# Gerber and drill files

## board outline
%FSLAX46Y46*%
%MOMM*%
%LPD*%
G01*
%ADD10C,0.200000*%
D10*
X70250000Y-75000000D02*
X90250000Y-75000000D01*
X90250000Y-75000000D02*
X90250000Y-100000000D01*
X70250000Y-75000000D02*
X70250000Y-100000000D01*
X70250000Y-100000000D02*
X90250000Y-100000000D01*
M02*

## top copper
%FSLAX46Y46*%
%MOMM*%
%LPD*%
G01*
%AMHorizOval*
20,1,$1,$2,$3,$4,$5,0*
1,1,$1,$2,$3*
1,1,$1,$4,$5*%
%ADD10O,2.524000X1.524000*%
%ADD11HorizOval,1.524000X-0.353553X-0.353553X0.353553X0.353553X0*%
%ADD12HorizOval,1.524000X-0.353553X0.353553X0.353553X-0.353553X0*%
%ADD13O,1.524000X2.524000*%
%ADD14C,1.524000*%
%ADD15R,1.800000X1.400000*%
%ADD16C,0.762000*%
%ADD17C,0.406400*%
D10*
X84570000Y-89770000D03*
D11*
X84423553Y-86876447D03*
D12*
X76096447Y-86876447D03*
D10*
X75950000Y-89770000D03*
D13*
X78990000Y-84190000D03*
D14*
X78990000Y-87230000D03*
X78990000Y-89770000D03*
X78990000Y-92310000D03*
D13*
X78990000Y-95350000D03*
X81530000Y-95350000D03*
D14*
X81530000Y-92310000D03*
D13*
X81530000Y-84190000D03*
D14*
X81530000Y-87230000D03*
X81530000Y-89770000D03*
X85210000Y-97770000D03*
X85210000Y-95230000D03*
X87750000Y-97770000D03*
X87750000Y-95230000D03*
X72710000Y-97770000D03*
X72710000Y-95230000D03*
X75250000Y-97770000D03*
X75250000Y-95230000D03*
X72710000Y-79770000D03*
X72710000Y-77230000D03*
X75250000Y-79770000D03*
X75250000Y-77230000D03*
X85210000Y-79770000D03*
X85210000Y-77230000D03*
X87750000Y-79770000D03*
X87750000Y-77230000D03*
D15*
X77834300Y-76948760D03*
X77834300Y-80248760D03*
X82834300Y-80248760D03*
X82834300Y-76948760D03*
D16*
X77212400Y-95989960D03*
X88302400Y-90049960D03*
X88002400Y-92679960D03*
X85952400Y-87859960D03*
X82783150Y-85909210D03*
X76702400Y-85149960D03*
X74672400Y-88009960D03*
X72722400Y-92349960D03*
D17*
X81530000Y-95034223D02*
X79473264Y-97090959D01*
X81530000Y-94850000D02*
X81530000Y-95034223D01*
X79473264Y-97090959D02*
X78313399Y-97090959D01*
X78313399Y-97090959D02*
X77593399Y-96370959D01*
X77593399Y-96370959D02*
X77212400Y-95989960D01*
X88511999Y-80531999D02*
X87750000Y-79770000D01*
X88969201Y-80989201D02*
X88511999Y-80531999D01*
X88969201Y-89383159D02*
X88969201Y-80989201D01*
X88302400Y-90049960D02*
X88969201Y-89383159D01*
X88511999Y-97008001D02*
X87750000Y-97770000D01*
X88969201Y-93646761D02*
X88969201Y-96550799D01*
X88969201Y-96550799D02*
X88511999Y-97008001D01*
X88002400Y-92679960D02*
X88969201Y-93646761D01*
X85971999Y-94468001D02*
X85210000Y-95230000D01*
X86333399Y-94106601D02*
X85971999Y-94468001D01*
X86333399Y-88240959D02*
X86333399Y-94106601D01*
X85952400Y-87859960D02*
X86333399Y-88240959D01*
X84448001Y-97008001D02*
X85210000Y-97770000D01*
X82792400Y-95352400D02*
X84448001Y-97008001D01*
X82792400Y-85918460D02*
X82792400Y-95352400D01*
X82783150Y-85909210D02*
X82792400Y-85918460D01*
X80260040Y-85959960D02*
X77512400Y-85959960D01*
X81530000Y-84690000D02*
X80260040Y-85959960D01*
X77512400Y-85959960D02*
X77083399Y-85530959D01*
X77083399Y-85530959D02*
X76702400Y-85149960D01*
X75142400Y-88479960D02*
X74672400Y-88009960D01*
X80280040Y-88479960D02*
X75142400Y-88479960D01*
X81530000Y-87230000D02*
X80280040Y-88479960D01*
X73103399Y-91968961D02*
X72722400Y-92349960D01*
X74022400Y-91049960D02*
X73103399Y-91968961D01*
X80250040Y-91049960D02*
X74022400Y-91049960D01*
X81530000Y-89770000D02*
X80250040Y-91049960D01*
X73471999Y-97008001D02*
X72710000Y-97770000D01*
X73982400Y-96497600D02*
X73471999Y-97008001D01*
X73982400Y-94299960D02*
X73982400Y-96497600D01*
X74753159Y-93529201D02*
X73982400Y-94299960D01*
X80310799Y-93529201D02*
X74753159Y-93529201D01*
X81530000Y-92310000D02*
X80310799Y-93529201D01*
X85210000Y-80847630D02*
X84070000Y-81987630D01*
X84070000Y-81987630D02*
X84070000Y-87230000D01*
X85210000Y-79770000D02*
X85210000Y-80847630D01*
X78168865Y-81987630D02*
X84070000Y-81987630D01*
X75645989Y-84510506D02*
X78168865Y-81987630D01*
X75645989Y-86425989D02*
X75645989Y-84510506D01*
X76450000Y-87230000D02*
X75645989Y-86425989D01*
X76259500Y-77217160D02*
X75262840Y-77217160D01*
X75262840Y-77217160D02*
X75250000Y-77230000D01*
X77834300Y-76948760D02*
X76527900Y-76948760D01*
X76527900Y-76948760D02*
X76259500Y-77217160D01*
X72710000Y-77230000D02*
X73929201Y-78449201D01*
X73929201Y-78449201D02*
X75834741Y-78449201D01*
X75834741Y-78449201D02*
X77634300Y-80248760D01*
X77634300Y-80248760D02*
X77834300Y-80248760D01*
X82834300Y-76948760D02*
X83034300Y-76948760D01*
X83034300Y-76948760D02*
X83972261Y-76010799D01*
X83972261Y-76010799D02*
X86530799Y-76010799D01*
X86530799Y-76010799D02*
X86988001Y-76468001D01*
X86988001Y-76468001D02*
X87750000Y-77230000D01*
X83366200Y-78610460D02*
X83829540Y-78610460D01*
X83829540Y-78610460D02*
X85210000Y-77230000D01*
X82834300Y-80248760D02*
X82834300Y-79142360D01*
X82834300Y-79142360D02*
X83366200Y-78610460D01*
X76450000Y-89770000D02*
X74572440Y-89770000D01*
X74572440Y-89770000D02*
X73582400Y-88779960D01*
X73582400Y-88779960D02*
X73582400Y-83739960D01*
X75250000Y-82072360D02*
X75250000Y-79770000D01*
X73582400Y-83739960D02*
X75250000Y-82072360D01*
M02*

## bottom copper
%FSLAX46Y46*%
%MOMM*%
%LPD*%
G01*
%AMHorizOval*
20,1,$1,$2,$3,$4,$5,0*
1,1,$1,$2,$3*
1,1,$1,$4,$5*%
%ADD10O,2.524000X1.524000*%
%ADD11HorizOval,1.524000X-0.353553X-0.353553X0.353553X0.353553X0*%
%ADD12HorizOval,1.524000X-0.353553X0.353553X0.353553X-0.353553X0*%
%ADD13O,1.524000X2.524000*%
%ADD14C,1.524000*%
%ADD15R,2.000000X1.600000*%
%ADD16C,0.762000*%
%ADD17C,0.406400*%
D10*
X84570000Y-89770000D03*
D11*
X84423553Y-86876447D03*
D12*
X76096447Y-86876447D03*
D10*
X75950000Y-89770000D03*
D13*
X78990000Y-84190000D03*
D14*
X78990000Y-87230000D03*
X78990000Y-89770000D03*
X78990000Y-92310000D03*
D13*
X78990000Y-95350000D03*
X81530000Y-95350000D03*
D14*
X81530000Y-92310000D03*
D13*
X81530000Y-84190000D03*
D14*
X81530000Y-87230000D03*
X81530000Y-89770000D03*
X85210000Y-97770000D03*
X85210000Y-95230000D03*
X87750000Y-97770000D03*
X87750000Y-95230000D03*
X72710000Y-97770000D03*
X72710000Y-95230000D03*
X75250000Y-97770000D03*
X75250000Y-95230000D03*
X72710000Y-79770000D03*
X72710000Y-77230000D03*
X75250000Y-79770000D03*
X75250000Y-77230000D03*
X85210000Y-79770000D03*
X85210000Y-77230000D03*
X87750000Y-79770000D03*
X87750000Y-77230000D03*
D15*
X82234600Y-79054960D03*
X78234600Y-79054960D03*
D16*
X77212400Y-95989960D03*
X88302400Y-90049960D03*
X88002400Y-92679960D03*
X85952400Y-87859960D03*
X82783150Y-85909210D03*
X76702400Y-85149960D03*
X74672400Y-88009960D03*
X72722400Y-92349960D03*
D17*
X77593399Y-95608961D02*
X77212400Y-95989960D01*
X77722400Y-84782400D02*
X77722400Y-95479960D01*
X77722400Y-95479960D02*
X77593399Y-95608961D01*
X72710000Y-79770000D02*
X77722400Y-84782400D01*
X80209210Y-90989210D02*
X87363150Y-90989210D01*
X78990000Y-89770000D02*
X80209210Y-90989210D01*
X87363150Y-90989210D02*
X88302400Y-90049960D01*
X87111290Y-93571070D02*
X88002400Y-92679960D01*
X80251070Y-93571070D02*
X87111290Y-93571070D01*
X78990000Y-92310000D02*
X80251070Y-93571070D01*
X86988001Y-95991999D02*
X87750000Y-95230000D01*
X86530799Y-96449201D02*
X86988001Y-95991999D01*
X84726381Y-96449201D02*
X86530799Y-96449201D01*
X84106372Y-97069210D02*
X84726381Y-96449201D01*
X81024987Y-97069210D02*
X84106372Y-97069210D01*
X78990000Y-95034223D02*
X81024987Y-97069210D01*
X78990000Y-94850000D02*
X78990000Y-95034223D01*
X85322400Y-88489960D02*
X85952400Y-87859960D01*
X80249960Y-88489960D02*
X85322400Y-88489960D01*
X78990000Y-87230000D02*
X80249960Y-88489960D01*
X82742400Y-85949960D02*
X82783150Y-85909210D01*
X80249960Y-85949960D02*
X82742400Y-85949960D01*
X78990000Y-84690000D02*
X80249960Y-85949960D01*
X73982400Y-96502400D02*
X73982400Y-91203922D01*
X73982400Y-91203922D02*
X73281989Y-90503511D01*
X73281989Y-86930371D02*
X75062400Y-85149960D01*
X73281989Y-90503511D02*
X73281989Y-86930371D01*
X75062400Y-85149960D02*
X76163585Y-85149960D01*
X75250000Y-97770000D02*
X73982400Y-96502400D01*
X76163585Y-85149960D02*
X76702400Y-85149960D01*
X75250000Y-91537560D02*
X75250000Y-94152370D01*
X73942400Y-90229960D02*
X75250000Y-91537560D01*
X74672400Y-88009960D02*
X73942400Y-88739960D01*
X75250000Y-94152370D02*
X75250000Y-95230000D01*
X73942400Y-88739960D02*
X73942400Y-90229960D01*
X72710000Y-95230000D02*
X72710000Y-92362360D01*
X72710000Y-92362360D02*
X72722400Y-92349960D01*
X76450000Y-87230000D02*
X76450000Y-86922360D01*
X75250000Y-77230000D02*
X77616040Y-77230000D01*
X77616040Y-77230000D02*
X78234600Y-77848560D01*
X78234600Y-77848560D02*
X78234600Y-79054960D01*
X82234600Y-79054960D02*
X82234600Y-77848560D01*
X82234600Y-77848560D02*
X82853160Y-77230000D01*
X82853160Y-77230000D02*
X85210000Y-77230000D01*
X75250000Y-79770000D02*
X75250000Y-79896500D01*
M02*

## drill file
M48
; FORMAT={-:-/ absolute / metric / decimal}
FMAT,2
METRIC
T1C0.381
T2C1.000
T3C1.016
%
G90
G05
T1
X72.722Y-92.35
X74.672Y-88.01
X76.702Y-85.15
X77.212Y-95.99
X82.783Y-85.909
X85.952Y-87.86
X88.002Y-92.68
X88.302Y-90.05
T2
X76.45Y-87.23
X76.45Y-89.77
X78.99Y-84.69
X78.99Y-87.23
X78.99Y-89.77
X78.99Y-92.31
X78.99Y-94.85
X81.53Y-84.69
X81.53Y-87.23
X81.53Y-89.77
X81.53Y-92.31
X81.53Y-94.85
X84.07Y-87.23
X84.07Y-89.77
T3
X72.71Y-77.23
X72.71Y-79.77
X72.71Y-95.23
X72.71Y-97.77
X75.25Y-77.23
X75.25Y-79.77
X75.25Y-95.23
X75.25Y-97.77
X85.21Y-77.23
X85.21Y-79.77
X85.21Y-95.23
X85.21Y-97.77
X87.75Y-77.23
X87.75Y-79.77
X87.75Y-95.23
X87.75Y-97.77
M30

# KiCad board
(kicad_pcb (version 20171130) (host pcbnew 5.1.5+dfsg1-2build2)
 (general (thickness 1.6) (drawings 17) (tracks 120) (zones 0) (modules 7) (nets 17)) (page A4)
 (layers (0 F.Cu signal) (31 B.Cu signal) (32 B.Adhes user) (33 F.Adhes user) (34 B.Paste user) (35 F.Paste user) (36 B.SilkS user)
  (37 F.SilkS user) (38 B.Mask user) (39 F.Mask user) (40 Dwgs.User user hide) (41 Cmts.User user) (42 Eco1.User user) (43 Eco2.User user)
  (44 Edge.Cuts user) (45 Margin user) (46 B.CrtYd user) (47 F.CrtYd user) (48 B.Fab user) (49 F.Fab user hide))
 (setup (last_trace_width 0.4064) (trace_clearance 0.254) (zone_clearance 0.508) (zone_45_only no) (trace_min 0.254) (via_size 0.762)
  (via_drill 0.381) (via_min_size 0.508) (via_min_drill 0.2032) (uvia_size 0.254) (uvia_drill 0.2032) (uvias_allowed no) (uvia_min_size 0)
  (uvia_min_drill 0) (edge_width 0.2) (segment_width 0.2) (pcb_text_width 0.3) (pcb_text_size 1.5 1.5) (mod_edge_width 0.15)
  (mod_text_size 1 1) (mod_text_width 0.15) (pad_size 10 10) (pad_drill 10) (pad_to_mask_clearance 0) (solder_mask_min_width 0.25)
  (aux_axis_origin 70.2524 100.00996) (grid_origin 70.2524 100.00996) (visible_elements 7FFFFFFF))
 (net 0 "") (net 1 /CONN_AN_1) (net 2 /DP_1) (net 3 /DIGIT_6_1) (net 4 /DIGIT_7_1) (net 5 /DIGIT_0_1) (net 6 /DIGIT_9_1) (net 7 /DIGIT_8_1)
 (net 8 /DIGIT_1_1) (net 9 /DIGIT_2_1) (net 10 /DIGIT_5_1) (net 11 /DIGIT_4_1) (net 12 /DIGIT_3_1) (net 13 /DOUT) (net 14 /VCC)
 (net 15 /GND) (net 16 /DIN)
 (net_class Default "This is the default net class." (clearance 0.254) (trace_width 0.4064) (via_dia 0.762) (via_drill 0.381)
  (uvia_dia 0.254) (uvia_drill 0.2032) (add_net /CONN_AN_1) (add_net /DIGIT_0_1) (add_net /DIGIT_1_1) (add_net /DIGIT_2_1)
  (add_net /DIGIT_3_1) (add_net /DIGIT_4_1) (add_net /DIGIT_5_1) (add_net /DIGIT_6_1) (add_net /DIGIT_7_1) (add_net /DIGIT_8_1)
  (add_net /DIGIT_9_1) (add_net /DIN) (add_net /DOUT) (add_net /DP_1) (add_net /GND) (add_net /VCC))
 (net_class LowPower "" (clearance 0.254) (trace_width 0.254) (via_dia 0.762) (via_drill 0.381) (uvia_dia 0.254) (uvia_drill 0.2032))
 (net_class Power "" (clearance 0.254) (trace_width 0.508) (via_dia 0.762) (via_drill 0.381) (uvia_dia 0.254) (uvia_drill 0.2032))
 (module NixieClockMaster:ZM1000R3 (layer F.Cu) (at 80.26 88.5 180)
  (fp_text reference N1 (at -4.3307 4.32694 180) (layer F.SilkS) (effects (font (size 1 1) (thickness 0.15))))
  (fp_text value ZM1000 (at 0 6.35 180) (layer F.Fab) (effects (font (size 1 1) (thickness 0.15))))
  (pad PR thru_hole oval (at -3.81 -1.27 180) (size 2.524 1.524) (drill 1 (offset -0.5 0)) (layers *.Cu *.Mask))
  (pad A1 thru_hole oval (at -3.81 1.27 225) (size 2.524 1.524) (drill 1 (offset -0.5 0)) (layers *.Cu *.Mask) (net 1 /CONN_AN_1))
  (pad A2 thru_hole oval (at 3.81 1.27 135) (size 2.524 1.524) (drill 1 (offset 0.5 0)) (layers *.Cu *.Mask) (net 1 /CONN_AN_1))
  (pad Kdp thru_hole oval (at 3.81 -1.27 180) (size 2.524 1.524) (drill 1 (offset 0.5 0)) (layers *.Cu *.Mask) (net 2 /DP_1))
  (pad K6 thru_hole oval (at 1.27 3.81 180) (size 1.524 2.524) (drill 1 (offset 0 0.5)) (layers *.Cu *.Mask) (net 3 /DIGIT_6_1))
  (pad K7 thru_hole circle (at 1.27 1.27 180) (size 1.524 1.524) (drill 1) (layers *.Cu *.Mask) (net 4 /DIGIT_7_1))
  (pad K0 thru_hole circle (at 1.27 -1.27 180) (size 1.524 1.524) (drill 1) (layers *.Cu *.Mask) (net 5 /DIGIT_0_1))
  (pad K9 thru_hole circle (at 1.27 -3.81 180) (size 1.524 1.524) (drill 1) (layers *.Cu *.Mask) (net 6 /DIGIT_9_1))
  (pad K8 thru_hole oval (at 1.27 -6.35 180) (size 1.524 2.524) (drill 1 (offset 0 -0.5)) (layers *.Cu *.Mask) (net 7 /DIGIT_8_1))
  (pad K1 thru_hole oval (at -1.27 -6.35 180) (size 1.524 2.524) (drill 1 (offset 0 -0.5)) (layers *.Cu *.Mask) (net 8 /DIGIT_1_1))
  (pad K2 thru_hole circle (at -1.27 -3.81 180) (size 1.524 1.524) (drill 1) (layers *.Cu *.Mask) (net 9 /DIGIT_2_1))
  (pad K5 thru_hole oval (at -1.27 3.81 180) (size 1.524 2.524) (drill 1 (offset 0 0.5)) (layers *.Cu *.Mask) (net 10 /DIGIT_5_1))
  (pad K4 thru_hole circle (at -1.27 1.27 180) (size 1.524 1.524) (drill 1) (layers *.Cu *.Mask) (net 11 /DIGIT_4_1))
  (pad K3 thru_hole circle (at -1.27 -1.27 180) (size 1.524 1.524) (drill 1) (layers *.Cu *.Mask) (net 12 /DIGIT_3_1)))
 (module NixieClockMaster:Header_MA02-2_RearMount (layer F.Cu) (at 87.75 96.5)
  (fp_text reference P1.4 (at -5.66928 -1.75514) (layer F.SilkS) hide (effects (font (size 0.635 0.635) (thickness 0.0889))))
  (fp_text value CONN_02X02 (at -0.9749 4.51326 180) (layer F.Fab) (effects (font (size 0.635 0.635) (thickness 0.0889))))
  (pad 1 thru_hole circle (at -2.54 1.27) (size 1.524 1.524) (drill 1.016) (layers *.Cu *.Mask F.Paste F.SilkS) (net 3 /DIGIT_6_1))
  (pad 2 thru_hole circle (at -2.54 -1.27) (size 1.524 1.524) (drill 1.016) (layers *.Cu *.Mask F.Paste F.SilkS) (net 4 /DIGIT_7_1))
  (pad 3 thru_hole circle (at 0 1.27) (size 1.524 1.524) (drill 1.016) (layers *.Cu *.Mask F.Paste F.SilkS) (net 6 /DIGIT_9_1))
  (pad 4 thru_hole circle (at 0 -1.27) (size 1.524 1.524) (drill 1.016) (layers *.Cu *.Mask F.Paste F.SilkS) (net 7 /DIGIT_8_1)))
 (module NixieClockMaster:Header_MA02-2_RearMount (layer F.Cu) (at 75.25 96.5)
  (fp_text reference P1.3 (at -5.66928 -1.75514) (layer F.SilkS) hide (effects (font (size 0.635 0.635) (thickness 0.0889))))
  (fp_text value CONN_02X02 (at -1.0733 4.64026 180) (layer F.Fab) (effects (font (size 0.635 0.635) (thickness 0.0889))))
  (pad 1 thru_hole circle (at -2.54 1.27) (size 1.524 1.524) (drill 1.016) (layers *.Cu *.Mask F.Paste F.SilkS) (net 9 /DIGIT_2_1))
  (pad 2 thru_hole circle (at -2.54 -1.27) (size 1.524 1.524) (drill 1.016) (layers *.Cu *.Mask F.Paste F.SilkS) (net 12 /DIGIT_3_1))
  (pad 3 thru_hole circle (at 0 1.27) (size 1.524 1.524) (drill 1.016) (layers *.Cu *.Mask F.Paste F.SilkS) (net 10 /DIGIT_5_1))
  (pad 4 thru_hole circle (at 0 -1.27) (size 1.524 1.524) (drill 1.016) (layers *.Cu *.Mask F.Paste F.SilkS) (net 11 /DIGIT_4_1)))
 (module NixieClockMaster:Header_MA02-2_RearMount (layer F.Cu) (at 75.25 78.5)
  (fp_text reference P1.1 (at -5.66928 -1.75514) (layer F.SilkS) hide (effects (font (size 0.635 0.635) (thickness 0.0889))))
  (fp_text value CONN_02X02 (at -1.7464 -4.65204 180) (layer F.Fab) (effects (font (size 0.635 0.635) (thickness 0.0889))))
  (pad 1 thru_hole circle (at -2.54 1.27) (size 1.524 1.524) (drill 1.016) (layers *.Cu *.Mask F.Paste F.SilkS) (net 8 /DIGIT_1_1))
  (pad 2 thru_hole circle (at -2.54 -1.27) (size 1.524 1.524) (drill 1.016) (layers *.Cu *.Mask F.Paste F.SilkS) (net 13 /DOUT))
  (pad 3 thru_hole circle (at 0 1.27) (size 1.524 1.524) (drill 1.016) (layers *.Cu *.Mask F.Paste F.SilkS) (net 2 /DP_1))
  (pad 4 thru_hole circle (at 0 -1.27) (size 1.524 1.524) (drill 1.016) (layers *.Cu *.Mask F.Paste F.SilkS) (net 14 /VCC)))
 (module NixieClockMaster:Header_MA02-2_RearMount (layer F.Cu) (at 87.75 78.5)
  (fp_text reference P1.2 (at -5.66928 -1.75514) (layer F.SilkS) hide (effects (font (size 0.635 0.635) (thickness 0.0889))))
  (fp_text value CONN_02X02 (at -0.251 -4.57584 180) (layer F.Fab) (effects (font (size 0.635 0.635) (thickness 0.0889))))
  (pad 1 thru_hole circle (at -2.54 1.27) (size 1.524 1.524) (drill 1.016) (layers *.Cu *.Mask F.Paste F.SilkS) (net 1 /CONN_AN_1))
  (pad 2 thru_hole circle (at -2.54 -1.27) (size 1.524 1.524) (drill 1.016) (layers *.Cu *.Mask F.Paste F.SilkS) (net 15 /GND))
  (pad 3 thru_hole circle (at 0 1.27) (size 1.524 1.524) (drill 1.016) (layers *.Cu *.Mask F.Paste F.SilkS) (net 5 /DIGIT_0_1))
  (pad 4 thru_hole circle (at 0 -1.27) (size 1.524 1.524) (drill 1.016) (layers *.Cu *.Mask F.Paste F.SilkS) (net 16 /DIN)))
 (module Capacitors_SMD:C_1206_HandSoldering (layer B.Cu) (at 80.2346 79.05496 180)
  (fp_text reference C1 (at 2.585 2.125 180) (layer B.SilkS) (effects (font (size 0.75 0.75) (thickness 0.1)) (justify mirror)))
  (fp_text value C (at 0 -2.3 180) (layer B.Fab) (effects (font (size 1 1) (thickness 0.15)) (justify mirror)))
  (pad 1 smd rect (at -2 0 180) (size 2 1.6) (layers B.Cu B.Paste B.Mask) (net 15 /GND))
  (pad 2 smd rect (at 2 0 180) (size 2 1.6) (layers B.Cu B.Paste B.Mask) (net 14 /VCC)))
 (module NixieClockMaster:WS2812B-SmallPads (layer F.Cu) (at 80.3343 78.59876 90)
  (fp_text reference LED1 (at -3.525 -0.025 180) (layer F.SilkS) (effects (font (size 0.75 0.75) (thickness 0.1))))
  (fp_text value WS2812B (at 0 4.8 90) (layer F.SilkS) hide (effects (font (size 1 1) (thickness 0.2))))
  (pad 1 smd rect (at 1.65 -2.5 90) (size 1.4 1.8) (layers F.Cu F.Paste F.Mask) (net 14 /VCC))
  (pad 2 smd rect (at -1.65 -2.5 90) (size 1.4 1.8) (layers F.Cu F.Paste F.Mask) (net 13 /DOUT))
  (pad 3 smd rect (at -1.65 2.5 90) (size 1.4 1.8) (layers F.Cu F.Paste F.Mask) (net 15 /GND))
  (pad 4 smd rect (at 1.65 2.5 90) (size 1.4 1.8) (layers F.Cu F.Paste F.Mask) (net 16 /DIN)))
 (gr_line (start 70.25 75) (end 90.25 75) (layer Edge.Cuts) (width 0.2))
 (gr_line (start 90.25 75) (end 90.25 100) (layer Edge.Cuts) (width 0.2))
 (gr_line (start 70.25 75) (end 70.25 100) (layer Edge.Cuts) (width 0.2))
 (gr_line (start 70.25 100) (end 90.25 100) (layer Edge.Cuts) (width 0.2))
 (via (at 77.2124 95.98996) (size 0.762) (drill 0.381) (layers F.Cu B.Cu) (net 8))
 (segment (start 81.53 95.034223) (end 79.473264 97.090959) (width 0.4064) (layer F.Cu) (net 8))
 (segment (start 81.53 94.85) (end 81.53 95.034223) (width 0.4064) (layer F.Cu) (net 8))
 (segment (start 79.473264 97.090959) (end 78.313399 97.090959) (width 0.4064) (layer F.Cu) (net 8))
 (segment (start 78.313399 97.090959) (end 77.593399 96.370959) (width 0.4064) (layer F.Cu) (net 8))
 (segment (start 77.593399 96.370959) (end 77.2124 95.98996) (width 0.4064) (layer F.Cu) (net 8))
 (segment (start 77.593399 95.608961) (end 77.2124 95.98996) (width 0.4064) (layer B.Cu) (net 8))
 (segment (start 77.7224 84.7824) (end 77.7224 95.47996) (width 0.4064) (layer B.Cu) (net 8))
 (segment (start 77.7224 95.47996) (end 77.593399 95.608961) (width 0.4064) (layer B.Cu) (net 8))
 (segment (start 72.71 79.77) (end 77.7224 84.7824) (width 0.4064) (layer B.Cu) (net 8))
 (segment (start 80.20921 90.98921) (end 87.36315 90.98921) (width 0.4064) (layer B.Cu) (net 5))
 (segment (start 78.99 89.77) (end 80.20921 90.98921) (width 0.4064) (layer B.Cu) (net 5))
 (via (at 88.3024 90.04996) (size 0.762) (drill 0.381) (layers F.Cu B.Cu) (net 5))
 (segment (start 87.36315 90.98921) (end 88.3024 90.04996) (width 0.4064) (layer B.Cu) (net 5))
 (segment (start 88.511999 80.531999) (end 87.75 79.77) (width 0.4064) (layer F.Cu) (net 5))
 (segment (start 88.969201 80.989201) (end 88.511999 80.531999) (width 0.4064) (layer F.Cu) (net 5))
 (segment (start 88.969201 89.383159) (end 88.969201 80.989201) (width 0.4064) (layer F.Cu) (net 5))
 (segment (start 88.3024 90.04996) (end 88.969201 89.383159) (width 0.4064) (layer F.Cu) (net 5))
 (via (at 88.0024 92.67996) (size 0.762) (drill 0.381) (layers F.Cu B.Cu) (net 6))
 (segment (start 88.511999 97.008001) (end 87.75 97.77) (width 0.4064) (layer F.Cu) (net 6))
 (segment (start 88.969201 93.646761) (end 88.969201 96.550799) (width 0.4064) (layer F.Cu) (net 6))
 (segment (start 88.969201 96.550799) (end 88.511999 97.008001) (width 0.4064) (layer F.Cu) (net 6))
 (segment (start 88.0024 92.67996) (end 88.969201 93.646761) (width 0.4064) (layer F.Cu) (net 6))
 (segment (start 87.11129 93.57107) (end 88.0024 92.67996) (width 0.4064) (layer B.Cu) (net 6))
 (segment (start 80.25107 93.57107) (end 87.11129 93.57107) (width 0.4064) (layer B.Cu) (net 6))
 (segment (start 78.99 92.31) (end 80.25107 93.57107) (width 0.4064) (layer B.Cu) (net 6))
 (segment (start 86.988001 95.991999) (end 87.75 95.23) (width 0.4064) (layer B.Cu) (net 7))
 (segment (start 86.530799 96.449201) (end 86.988001 95.991999) (width 0.4064) (layer B.Cu) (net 7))
 (segment (start 84.726381 96.449201) (end 86.530799 96.449201) (width 0.4064) (layer B.Cu) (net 7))
 (segment (start 84.106372 97.06921) (end 84.726381 96.449201) (width 0.4064) (layer B.Cu) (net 7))
 (segment (start 81.024987 97.06921) (end 84.106372 97.06921) (width 0.4064) (layer B.Cu) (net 7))
 (segment (start 78.99 95.034223) (end 81.024987 97.06921) (width 0.4064) (layer B.Cu) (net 7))
 (segment (start 78.99 94.85) (end 78.99 95.034223) (width 0.4064) (layer B.Cu) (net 7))
 (via (at 85.9524 87.85996) (size 0.762) (drill 0.381) (layers F.Cu B.Cu) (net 4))
 (segment (start 85.971999 94.468001) (end 85.21 95.23) (width 0.4064) (layer F.Cu) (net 4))
 (segment (start 86.333399 94.106601) (end 85.971999 94.468001) (width 0.4064) (layer F.Cu) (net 4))
 (segment (start 86.333399 88.240959) (end 86.333399 94.106601) (width 0.4064) (layer F.Cu) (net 4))
 (segment (start 85.9524 87.85996) (end 86.333399 88.240959) (width 0.4064) (layer F.Cu) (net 4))
 (segment (start 85.3224 88.48996) (end 85.9524 87.85996) (width 0.4064) (layer B.Cu) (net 4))
 (segment (start 80.24996 88.48996) (end 85.3224 88.48996) (width 0.4064) (layer B.Cu) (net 4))
 (segment (start 78.99 87.23) (end 80.24996 88.48996) (width 0.4064) (layer B.Cu) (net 4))
 (via (at 82.78315 85.90921) (size 0.762) (drill 0.381) (layers F.Cu B.Cu) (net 3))
 (segment (start 84.448001 97.008001) (end 85.21 97.77) (width 0.4064) (layer F.Cu) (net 3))
 (segment (start 82.7924 95.3524) (end 84.448001 97.008001) (width 0.4064) (layer F.Cu) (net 3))
 (segment (start 82.7924 85.91846) (end 82.7924 95.3524) (width 0.4064) (layer F.Cu) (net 3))
 (segment (start 82.78315 85.90921) (end 82.7924 85.91846) (width 0.4064) (layer F.Cu) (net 3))
 (segment (start 82.7424 85.94996) (end 82.78315 85.90921) (width 0.4064) (layer B.Cu) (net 3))
 (segment (start 80.24996 85.94996) (end 82.7424 85.94996) (width 0.4064) (layer B.Cu) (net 3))
 (segment (start 78.99 84.69) (end 80.24996 85.94996) (width 0.4064) (layer B.Cu) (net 3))
 (via (at 76.7024 85.14996) (size 0.762) (drill 0.381) (layers F.Cu B.Cu) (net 10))
 (segment (start 80.26004 85.95996) (end 77.5124 85.95996) (width 0.4064) (layer F.Cu) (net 10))
 (segment (start 73.9824 96.5024) (end 73.9824 91.203922) (width 0.4064) (layer B.Cu) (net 10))
 (segment (start 81.53 84.69) (end 80.26004 85.95996) (width 0.4064) (layer F.Cu) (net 10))
 (segment (start 77.5124 85.95996) (end 77.083399 85.530959) (width 0.4064) (layer F.Cu) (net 10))
 (segment (start 73.9824 91.203922) (end 73.281989 90.503511) (width 0.4064) (layer B.Cu) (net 10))
 (segment (start 73.281989 86.930371) (end 75.0624 85.14996) (width 0.4064) (layer B.Cu) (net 10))
 (segment (start 77.083399 85.530959) (end 76.7024 85.14996) (width 0.4064) (layer F.Cu) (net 10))
 (segment (start 73.281989 90.503511) (end 73.281989 86.930371) (width 0.4064) (layer B.Cu) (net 10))
 (segment (start 75.0624 85.14996) (end 76.163585 85.14996) (width 0.4064) (layer B.Cu) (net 10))
 (segment (start 75.25 97.77) (end 73.9824 96.5024) (width 0.4064) (layer B.Cu) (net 10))
 (segment (start 76.163585 85.14996) (end 76.7024 85.14996) (width 0.4064) (layer B.Cu) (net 10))
 (via (at 74.6724 88.00996) (size 0.762) (drill 0.381) (layers F.Cu B.Cu) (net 11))
 (segment (start 75.25 91.53756) (end 75.25 94.15237) (width 0.4064) (layer B.Cu) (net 11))
 (segment (start 73.9424 90.22996) (end 75.25 91.53756) (width 0.4064) (layer B.Cu) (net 11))
 (segment (start 74.6724 88.00996) (end 73.9424 88.73996) (width 0.4064) (layer B.Cu) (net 11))
 (segment (start 75.25 94.15237) (end 75.25 95.23) (width 0.4064) (layer B.Cu) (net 11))
 (segment (start 73.9424 88.73996) (end 73.9424 90.22996) (width 0.4064) (layer B.Cu) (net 11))
 (segment (start 75.1424 88.47996) (end 74.6724 88.00996) (width 0.4064) (layer F.Cu) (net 11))
 (segment (start 80.28004 88.47996) (end 75.1424 88.47996) (width 0.4064) (layer F.Cu) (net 11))
 (segment (start 81.53 87.23) (end 80.28004 88.47996) (width 0.4064) (layer F.Cu) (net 11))
 (via (at 72.7224 92.34996) (size 0.762) (drill 0.381) (layers F.Cu B.Cu) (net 12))
 (segment (start 72.71 95.23) (end 72.71 92.36236) (width 0.4064) (layer B.Cu) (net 12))
 (segment (start 72.71 92.36236) (end 72.7224 92.34996) (width 0.4064) (layer B.Cu) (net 12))
 (segment (start 73.103399 91.968961) (end 72.7224 92.34996) (width 0.4064) (layer F.Cu) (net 12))
 (segment (start 74.0224 91.04996) (end 73.103399 91.968961) (width 0.4064) (layer F.Cu) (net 12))
 (segment (start 80.25004 91.04996) (end 74.0224 91.04996) (width 0.4064) (layer F.Cu) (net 12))
 (segment (start 81.53 89.77) (end 80.25004 91.04996) (width 0.4064) (layer F.Cu) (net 12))
 (segment (start 73.471999 97.008001) (end 72.71 97.77) (width 0.4064) (layer F.Cu) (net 9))
 (segment (start 73.9824 96.4976) (end 73.471999 97.008001) (width 0.4064) (layer F.Cu) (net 9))
 (segment (start 73.9824 94.29996) (end 73.9824 96.4976) (width 0.4064) (layer F.Cu) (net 9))
 (segment (start 74.753159 93.529201) (end 73.9824 94.29996) (width 0.4064) (layer F.Cu) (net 9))
 (segment (start 80.310799 93.529201) (end 74.753159 93.529201) (width 0.4064) (layer F.Cu) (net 9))
 (segment (start 81.53 92.31) (end 80.310799 93.529201) (width 0.4064) (layer F.Cu) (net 9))
 (segment (start 85.21 80.84763) (end 84.07 81.98763) (width 0.4064) (layer F.Cu) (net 1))
 (segment (start 84.07 81.98763) (end 84.07 87.23) (width 0.4064) (layer F.Cu) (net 1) (status 20))
 (segment (start 85.21 79.77) (end 85.21 80.84763) (width 0.4064) (layer F.Cu) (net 1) (status 10))
 (segment (start 76.45 87.23) (end 76.45 86.92236) (width 0.4064) (layer B.Cu) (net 1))
 (segment (start 78.168865 81.98763) (end 84.07 81.98763) (width 0.4064) (layer F.Cu) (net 1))
 (segment (start 75.645989 84.510506) (end 78.168865 81.98763) (width 0.4064) (layer F.Cu) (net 1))
 (segment (start 75.645989 86.425989) (end 75.645989 84.510506) (width 0.4064) (layer F.Cu) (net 1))
 (segment (start 76.45 87.23) (end 75.645989 86.425989) (width 0.4064) (layer F.Cu) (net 1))
 (segment (start 76.2595 77.21716) (end 75.26284 77.21716) (width 0.4064) (layer F.Cu) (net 14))
 (segment (start 75.26284 77.21716) (end 75.25 77.23) (width 0.4064) (layer F.Cu) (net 14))
 (segment (start 77.8343 76.94876) (end 76.5279 76.94876) (width 0.4064) (layer F.Cu) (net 14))
 (segment (start 76.5279 76.94876) (end 76.2595 77.21716) (width 0.4064) (layer F.Cu) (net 14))
 (segment (start 75.25 77.23) (end 77.61604 77.23) (width 0.4064) (layer B.Cu) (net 14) (status 10))
 (segment (start 77.61604 77.23) (end 78.2346 77.84856) (width 0.4064) (layer B.Cu) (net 14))
 (segment (start 78.2346 77.84856) (end 78.2346 79.05496) (width 0.4064) (layer B.Cu) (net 14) (status 20))
 (segment (start 72.71 77.23) (end 73.929201 78.449201) (width 0.4064) (layer F.Cu) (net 13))
 (segment (start 73.929201 78.449201) (end 75.834741 78.449201) (width 0.4064) (layer F.Cu) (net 13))
 (segment (start 75.834741 78.449201) (end 77.6343 80.24876) (width 0.4064) (layer F.Cu) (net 13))
 (segment (start 77.6343 80.24876) (end 77.8343 80.24876) (width 0.4064) (layer F.Cu) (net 13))
 (segment (start 82.8343 76.94876) (end 83.0343 76.94876) (width 0.4064) (layer F.Cu) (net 16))
 (segment (start 83.0343 76.94876) (end 83.972261 76.010799) (width 0.4064) (layer F.Cu) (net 16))
 (segment (start 83.972261 76.010799) (end 86.530799 76.010799) (width 0.4064) (layer F.Cu) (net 16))
 (segment (start 86.530799 76.010799) (end 86.988001 76.468001) (width 0.4064) (layer F.Cu) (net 16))
 (segment (start 86.988001 76.468001) (end 87.75 77.23) (width 0.4064) (layer F.Cu) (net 16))
 (segment (start 83.3662 78.61046) (end 83.82954 78.61046) (width 0.4064) (layer F.Cu) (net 15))
 (segment (start 83.82954 78.61046) (end 85.21 77.23) (width 0.4064) (layer F.Cu) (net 15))
 (segment (start 82.8343 80.24876) (end 82.8343 79.14236) (width 0.4064) (layer F.Cu) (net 15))
 (segment (start 82.8343 79.14236) (end 83.3662 78.61046) (width 0.4064) (layer F.Cu) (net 15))
 (segment (start 82.2346 79.05496) (end 82.2346 77.84856) (width 0.4064) (layer B.Cu) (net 15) (status 10))
 (segment (start 82.2346 77.84856) (end 82.85316 77.23) (width 0.4064) (layer B.Cu) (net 15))
 (segment (start 82.85316 77.23) (end 85.21 77.23) (width 0.4064) (layer B.Cu) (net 15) (status 20))
 (segment (start 75.25 79.77) (end 75.25 79.8965) (width 0.4064) (layer B.Cu) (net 2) (status 30))
 (segment (start 76.45 89.77) (end 74.57244 89.77) (width 0.4064) (layer F.Cu) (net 2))
 (segment (start 74.57244 89.77) (end 73.5824 88.77996) (width 0.4064) (layer F.Cu) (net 2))
 (segment (start 73.5824 88.77996) (end 73.5824 83.73996) (width 0.4064) (layer F.Cu) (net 2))
 (segment (start 75.25 82.07236) (end 75.25 79.77) (width 0.4064) (layer F.Cu) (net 2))
 (segment (start 73.5824 83.73996) (end 75.25 82.07236) (width 0.4064) (layer F.Cu) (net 2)))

